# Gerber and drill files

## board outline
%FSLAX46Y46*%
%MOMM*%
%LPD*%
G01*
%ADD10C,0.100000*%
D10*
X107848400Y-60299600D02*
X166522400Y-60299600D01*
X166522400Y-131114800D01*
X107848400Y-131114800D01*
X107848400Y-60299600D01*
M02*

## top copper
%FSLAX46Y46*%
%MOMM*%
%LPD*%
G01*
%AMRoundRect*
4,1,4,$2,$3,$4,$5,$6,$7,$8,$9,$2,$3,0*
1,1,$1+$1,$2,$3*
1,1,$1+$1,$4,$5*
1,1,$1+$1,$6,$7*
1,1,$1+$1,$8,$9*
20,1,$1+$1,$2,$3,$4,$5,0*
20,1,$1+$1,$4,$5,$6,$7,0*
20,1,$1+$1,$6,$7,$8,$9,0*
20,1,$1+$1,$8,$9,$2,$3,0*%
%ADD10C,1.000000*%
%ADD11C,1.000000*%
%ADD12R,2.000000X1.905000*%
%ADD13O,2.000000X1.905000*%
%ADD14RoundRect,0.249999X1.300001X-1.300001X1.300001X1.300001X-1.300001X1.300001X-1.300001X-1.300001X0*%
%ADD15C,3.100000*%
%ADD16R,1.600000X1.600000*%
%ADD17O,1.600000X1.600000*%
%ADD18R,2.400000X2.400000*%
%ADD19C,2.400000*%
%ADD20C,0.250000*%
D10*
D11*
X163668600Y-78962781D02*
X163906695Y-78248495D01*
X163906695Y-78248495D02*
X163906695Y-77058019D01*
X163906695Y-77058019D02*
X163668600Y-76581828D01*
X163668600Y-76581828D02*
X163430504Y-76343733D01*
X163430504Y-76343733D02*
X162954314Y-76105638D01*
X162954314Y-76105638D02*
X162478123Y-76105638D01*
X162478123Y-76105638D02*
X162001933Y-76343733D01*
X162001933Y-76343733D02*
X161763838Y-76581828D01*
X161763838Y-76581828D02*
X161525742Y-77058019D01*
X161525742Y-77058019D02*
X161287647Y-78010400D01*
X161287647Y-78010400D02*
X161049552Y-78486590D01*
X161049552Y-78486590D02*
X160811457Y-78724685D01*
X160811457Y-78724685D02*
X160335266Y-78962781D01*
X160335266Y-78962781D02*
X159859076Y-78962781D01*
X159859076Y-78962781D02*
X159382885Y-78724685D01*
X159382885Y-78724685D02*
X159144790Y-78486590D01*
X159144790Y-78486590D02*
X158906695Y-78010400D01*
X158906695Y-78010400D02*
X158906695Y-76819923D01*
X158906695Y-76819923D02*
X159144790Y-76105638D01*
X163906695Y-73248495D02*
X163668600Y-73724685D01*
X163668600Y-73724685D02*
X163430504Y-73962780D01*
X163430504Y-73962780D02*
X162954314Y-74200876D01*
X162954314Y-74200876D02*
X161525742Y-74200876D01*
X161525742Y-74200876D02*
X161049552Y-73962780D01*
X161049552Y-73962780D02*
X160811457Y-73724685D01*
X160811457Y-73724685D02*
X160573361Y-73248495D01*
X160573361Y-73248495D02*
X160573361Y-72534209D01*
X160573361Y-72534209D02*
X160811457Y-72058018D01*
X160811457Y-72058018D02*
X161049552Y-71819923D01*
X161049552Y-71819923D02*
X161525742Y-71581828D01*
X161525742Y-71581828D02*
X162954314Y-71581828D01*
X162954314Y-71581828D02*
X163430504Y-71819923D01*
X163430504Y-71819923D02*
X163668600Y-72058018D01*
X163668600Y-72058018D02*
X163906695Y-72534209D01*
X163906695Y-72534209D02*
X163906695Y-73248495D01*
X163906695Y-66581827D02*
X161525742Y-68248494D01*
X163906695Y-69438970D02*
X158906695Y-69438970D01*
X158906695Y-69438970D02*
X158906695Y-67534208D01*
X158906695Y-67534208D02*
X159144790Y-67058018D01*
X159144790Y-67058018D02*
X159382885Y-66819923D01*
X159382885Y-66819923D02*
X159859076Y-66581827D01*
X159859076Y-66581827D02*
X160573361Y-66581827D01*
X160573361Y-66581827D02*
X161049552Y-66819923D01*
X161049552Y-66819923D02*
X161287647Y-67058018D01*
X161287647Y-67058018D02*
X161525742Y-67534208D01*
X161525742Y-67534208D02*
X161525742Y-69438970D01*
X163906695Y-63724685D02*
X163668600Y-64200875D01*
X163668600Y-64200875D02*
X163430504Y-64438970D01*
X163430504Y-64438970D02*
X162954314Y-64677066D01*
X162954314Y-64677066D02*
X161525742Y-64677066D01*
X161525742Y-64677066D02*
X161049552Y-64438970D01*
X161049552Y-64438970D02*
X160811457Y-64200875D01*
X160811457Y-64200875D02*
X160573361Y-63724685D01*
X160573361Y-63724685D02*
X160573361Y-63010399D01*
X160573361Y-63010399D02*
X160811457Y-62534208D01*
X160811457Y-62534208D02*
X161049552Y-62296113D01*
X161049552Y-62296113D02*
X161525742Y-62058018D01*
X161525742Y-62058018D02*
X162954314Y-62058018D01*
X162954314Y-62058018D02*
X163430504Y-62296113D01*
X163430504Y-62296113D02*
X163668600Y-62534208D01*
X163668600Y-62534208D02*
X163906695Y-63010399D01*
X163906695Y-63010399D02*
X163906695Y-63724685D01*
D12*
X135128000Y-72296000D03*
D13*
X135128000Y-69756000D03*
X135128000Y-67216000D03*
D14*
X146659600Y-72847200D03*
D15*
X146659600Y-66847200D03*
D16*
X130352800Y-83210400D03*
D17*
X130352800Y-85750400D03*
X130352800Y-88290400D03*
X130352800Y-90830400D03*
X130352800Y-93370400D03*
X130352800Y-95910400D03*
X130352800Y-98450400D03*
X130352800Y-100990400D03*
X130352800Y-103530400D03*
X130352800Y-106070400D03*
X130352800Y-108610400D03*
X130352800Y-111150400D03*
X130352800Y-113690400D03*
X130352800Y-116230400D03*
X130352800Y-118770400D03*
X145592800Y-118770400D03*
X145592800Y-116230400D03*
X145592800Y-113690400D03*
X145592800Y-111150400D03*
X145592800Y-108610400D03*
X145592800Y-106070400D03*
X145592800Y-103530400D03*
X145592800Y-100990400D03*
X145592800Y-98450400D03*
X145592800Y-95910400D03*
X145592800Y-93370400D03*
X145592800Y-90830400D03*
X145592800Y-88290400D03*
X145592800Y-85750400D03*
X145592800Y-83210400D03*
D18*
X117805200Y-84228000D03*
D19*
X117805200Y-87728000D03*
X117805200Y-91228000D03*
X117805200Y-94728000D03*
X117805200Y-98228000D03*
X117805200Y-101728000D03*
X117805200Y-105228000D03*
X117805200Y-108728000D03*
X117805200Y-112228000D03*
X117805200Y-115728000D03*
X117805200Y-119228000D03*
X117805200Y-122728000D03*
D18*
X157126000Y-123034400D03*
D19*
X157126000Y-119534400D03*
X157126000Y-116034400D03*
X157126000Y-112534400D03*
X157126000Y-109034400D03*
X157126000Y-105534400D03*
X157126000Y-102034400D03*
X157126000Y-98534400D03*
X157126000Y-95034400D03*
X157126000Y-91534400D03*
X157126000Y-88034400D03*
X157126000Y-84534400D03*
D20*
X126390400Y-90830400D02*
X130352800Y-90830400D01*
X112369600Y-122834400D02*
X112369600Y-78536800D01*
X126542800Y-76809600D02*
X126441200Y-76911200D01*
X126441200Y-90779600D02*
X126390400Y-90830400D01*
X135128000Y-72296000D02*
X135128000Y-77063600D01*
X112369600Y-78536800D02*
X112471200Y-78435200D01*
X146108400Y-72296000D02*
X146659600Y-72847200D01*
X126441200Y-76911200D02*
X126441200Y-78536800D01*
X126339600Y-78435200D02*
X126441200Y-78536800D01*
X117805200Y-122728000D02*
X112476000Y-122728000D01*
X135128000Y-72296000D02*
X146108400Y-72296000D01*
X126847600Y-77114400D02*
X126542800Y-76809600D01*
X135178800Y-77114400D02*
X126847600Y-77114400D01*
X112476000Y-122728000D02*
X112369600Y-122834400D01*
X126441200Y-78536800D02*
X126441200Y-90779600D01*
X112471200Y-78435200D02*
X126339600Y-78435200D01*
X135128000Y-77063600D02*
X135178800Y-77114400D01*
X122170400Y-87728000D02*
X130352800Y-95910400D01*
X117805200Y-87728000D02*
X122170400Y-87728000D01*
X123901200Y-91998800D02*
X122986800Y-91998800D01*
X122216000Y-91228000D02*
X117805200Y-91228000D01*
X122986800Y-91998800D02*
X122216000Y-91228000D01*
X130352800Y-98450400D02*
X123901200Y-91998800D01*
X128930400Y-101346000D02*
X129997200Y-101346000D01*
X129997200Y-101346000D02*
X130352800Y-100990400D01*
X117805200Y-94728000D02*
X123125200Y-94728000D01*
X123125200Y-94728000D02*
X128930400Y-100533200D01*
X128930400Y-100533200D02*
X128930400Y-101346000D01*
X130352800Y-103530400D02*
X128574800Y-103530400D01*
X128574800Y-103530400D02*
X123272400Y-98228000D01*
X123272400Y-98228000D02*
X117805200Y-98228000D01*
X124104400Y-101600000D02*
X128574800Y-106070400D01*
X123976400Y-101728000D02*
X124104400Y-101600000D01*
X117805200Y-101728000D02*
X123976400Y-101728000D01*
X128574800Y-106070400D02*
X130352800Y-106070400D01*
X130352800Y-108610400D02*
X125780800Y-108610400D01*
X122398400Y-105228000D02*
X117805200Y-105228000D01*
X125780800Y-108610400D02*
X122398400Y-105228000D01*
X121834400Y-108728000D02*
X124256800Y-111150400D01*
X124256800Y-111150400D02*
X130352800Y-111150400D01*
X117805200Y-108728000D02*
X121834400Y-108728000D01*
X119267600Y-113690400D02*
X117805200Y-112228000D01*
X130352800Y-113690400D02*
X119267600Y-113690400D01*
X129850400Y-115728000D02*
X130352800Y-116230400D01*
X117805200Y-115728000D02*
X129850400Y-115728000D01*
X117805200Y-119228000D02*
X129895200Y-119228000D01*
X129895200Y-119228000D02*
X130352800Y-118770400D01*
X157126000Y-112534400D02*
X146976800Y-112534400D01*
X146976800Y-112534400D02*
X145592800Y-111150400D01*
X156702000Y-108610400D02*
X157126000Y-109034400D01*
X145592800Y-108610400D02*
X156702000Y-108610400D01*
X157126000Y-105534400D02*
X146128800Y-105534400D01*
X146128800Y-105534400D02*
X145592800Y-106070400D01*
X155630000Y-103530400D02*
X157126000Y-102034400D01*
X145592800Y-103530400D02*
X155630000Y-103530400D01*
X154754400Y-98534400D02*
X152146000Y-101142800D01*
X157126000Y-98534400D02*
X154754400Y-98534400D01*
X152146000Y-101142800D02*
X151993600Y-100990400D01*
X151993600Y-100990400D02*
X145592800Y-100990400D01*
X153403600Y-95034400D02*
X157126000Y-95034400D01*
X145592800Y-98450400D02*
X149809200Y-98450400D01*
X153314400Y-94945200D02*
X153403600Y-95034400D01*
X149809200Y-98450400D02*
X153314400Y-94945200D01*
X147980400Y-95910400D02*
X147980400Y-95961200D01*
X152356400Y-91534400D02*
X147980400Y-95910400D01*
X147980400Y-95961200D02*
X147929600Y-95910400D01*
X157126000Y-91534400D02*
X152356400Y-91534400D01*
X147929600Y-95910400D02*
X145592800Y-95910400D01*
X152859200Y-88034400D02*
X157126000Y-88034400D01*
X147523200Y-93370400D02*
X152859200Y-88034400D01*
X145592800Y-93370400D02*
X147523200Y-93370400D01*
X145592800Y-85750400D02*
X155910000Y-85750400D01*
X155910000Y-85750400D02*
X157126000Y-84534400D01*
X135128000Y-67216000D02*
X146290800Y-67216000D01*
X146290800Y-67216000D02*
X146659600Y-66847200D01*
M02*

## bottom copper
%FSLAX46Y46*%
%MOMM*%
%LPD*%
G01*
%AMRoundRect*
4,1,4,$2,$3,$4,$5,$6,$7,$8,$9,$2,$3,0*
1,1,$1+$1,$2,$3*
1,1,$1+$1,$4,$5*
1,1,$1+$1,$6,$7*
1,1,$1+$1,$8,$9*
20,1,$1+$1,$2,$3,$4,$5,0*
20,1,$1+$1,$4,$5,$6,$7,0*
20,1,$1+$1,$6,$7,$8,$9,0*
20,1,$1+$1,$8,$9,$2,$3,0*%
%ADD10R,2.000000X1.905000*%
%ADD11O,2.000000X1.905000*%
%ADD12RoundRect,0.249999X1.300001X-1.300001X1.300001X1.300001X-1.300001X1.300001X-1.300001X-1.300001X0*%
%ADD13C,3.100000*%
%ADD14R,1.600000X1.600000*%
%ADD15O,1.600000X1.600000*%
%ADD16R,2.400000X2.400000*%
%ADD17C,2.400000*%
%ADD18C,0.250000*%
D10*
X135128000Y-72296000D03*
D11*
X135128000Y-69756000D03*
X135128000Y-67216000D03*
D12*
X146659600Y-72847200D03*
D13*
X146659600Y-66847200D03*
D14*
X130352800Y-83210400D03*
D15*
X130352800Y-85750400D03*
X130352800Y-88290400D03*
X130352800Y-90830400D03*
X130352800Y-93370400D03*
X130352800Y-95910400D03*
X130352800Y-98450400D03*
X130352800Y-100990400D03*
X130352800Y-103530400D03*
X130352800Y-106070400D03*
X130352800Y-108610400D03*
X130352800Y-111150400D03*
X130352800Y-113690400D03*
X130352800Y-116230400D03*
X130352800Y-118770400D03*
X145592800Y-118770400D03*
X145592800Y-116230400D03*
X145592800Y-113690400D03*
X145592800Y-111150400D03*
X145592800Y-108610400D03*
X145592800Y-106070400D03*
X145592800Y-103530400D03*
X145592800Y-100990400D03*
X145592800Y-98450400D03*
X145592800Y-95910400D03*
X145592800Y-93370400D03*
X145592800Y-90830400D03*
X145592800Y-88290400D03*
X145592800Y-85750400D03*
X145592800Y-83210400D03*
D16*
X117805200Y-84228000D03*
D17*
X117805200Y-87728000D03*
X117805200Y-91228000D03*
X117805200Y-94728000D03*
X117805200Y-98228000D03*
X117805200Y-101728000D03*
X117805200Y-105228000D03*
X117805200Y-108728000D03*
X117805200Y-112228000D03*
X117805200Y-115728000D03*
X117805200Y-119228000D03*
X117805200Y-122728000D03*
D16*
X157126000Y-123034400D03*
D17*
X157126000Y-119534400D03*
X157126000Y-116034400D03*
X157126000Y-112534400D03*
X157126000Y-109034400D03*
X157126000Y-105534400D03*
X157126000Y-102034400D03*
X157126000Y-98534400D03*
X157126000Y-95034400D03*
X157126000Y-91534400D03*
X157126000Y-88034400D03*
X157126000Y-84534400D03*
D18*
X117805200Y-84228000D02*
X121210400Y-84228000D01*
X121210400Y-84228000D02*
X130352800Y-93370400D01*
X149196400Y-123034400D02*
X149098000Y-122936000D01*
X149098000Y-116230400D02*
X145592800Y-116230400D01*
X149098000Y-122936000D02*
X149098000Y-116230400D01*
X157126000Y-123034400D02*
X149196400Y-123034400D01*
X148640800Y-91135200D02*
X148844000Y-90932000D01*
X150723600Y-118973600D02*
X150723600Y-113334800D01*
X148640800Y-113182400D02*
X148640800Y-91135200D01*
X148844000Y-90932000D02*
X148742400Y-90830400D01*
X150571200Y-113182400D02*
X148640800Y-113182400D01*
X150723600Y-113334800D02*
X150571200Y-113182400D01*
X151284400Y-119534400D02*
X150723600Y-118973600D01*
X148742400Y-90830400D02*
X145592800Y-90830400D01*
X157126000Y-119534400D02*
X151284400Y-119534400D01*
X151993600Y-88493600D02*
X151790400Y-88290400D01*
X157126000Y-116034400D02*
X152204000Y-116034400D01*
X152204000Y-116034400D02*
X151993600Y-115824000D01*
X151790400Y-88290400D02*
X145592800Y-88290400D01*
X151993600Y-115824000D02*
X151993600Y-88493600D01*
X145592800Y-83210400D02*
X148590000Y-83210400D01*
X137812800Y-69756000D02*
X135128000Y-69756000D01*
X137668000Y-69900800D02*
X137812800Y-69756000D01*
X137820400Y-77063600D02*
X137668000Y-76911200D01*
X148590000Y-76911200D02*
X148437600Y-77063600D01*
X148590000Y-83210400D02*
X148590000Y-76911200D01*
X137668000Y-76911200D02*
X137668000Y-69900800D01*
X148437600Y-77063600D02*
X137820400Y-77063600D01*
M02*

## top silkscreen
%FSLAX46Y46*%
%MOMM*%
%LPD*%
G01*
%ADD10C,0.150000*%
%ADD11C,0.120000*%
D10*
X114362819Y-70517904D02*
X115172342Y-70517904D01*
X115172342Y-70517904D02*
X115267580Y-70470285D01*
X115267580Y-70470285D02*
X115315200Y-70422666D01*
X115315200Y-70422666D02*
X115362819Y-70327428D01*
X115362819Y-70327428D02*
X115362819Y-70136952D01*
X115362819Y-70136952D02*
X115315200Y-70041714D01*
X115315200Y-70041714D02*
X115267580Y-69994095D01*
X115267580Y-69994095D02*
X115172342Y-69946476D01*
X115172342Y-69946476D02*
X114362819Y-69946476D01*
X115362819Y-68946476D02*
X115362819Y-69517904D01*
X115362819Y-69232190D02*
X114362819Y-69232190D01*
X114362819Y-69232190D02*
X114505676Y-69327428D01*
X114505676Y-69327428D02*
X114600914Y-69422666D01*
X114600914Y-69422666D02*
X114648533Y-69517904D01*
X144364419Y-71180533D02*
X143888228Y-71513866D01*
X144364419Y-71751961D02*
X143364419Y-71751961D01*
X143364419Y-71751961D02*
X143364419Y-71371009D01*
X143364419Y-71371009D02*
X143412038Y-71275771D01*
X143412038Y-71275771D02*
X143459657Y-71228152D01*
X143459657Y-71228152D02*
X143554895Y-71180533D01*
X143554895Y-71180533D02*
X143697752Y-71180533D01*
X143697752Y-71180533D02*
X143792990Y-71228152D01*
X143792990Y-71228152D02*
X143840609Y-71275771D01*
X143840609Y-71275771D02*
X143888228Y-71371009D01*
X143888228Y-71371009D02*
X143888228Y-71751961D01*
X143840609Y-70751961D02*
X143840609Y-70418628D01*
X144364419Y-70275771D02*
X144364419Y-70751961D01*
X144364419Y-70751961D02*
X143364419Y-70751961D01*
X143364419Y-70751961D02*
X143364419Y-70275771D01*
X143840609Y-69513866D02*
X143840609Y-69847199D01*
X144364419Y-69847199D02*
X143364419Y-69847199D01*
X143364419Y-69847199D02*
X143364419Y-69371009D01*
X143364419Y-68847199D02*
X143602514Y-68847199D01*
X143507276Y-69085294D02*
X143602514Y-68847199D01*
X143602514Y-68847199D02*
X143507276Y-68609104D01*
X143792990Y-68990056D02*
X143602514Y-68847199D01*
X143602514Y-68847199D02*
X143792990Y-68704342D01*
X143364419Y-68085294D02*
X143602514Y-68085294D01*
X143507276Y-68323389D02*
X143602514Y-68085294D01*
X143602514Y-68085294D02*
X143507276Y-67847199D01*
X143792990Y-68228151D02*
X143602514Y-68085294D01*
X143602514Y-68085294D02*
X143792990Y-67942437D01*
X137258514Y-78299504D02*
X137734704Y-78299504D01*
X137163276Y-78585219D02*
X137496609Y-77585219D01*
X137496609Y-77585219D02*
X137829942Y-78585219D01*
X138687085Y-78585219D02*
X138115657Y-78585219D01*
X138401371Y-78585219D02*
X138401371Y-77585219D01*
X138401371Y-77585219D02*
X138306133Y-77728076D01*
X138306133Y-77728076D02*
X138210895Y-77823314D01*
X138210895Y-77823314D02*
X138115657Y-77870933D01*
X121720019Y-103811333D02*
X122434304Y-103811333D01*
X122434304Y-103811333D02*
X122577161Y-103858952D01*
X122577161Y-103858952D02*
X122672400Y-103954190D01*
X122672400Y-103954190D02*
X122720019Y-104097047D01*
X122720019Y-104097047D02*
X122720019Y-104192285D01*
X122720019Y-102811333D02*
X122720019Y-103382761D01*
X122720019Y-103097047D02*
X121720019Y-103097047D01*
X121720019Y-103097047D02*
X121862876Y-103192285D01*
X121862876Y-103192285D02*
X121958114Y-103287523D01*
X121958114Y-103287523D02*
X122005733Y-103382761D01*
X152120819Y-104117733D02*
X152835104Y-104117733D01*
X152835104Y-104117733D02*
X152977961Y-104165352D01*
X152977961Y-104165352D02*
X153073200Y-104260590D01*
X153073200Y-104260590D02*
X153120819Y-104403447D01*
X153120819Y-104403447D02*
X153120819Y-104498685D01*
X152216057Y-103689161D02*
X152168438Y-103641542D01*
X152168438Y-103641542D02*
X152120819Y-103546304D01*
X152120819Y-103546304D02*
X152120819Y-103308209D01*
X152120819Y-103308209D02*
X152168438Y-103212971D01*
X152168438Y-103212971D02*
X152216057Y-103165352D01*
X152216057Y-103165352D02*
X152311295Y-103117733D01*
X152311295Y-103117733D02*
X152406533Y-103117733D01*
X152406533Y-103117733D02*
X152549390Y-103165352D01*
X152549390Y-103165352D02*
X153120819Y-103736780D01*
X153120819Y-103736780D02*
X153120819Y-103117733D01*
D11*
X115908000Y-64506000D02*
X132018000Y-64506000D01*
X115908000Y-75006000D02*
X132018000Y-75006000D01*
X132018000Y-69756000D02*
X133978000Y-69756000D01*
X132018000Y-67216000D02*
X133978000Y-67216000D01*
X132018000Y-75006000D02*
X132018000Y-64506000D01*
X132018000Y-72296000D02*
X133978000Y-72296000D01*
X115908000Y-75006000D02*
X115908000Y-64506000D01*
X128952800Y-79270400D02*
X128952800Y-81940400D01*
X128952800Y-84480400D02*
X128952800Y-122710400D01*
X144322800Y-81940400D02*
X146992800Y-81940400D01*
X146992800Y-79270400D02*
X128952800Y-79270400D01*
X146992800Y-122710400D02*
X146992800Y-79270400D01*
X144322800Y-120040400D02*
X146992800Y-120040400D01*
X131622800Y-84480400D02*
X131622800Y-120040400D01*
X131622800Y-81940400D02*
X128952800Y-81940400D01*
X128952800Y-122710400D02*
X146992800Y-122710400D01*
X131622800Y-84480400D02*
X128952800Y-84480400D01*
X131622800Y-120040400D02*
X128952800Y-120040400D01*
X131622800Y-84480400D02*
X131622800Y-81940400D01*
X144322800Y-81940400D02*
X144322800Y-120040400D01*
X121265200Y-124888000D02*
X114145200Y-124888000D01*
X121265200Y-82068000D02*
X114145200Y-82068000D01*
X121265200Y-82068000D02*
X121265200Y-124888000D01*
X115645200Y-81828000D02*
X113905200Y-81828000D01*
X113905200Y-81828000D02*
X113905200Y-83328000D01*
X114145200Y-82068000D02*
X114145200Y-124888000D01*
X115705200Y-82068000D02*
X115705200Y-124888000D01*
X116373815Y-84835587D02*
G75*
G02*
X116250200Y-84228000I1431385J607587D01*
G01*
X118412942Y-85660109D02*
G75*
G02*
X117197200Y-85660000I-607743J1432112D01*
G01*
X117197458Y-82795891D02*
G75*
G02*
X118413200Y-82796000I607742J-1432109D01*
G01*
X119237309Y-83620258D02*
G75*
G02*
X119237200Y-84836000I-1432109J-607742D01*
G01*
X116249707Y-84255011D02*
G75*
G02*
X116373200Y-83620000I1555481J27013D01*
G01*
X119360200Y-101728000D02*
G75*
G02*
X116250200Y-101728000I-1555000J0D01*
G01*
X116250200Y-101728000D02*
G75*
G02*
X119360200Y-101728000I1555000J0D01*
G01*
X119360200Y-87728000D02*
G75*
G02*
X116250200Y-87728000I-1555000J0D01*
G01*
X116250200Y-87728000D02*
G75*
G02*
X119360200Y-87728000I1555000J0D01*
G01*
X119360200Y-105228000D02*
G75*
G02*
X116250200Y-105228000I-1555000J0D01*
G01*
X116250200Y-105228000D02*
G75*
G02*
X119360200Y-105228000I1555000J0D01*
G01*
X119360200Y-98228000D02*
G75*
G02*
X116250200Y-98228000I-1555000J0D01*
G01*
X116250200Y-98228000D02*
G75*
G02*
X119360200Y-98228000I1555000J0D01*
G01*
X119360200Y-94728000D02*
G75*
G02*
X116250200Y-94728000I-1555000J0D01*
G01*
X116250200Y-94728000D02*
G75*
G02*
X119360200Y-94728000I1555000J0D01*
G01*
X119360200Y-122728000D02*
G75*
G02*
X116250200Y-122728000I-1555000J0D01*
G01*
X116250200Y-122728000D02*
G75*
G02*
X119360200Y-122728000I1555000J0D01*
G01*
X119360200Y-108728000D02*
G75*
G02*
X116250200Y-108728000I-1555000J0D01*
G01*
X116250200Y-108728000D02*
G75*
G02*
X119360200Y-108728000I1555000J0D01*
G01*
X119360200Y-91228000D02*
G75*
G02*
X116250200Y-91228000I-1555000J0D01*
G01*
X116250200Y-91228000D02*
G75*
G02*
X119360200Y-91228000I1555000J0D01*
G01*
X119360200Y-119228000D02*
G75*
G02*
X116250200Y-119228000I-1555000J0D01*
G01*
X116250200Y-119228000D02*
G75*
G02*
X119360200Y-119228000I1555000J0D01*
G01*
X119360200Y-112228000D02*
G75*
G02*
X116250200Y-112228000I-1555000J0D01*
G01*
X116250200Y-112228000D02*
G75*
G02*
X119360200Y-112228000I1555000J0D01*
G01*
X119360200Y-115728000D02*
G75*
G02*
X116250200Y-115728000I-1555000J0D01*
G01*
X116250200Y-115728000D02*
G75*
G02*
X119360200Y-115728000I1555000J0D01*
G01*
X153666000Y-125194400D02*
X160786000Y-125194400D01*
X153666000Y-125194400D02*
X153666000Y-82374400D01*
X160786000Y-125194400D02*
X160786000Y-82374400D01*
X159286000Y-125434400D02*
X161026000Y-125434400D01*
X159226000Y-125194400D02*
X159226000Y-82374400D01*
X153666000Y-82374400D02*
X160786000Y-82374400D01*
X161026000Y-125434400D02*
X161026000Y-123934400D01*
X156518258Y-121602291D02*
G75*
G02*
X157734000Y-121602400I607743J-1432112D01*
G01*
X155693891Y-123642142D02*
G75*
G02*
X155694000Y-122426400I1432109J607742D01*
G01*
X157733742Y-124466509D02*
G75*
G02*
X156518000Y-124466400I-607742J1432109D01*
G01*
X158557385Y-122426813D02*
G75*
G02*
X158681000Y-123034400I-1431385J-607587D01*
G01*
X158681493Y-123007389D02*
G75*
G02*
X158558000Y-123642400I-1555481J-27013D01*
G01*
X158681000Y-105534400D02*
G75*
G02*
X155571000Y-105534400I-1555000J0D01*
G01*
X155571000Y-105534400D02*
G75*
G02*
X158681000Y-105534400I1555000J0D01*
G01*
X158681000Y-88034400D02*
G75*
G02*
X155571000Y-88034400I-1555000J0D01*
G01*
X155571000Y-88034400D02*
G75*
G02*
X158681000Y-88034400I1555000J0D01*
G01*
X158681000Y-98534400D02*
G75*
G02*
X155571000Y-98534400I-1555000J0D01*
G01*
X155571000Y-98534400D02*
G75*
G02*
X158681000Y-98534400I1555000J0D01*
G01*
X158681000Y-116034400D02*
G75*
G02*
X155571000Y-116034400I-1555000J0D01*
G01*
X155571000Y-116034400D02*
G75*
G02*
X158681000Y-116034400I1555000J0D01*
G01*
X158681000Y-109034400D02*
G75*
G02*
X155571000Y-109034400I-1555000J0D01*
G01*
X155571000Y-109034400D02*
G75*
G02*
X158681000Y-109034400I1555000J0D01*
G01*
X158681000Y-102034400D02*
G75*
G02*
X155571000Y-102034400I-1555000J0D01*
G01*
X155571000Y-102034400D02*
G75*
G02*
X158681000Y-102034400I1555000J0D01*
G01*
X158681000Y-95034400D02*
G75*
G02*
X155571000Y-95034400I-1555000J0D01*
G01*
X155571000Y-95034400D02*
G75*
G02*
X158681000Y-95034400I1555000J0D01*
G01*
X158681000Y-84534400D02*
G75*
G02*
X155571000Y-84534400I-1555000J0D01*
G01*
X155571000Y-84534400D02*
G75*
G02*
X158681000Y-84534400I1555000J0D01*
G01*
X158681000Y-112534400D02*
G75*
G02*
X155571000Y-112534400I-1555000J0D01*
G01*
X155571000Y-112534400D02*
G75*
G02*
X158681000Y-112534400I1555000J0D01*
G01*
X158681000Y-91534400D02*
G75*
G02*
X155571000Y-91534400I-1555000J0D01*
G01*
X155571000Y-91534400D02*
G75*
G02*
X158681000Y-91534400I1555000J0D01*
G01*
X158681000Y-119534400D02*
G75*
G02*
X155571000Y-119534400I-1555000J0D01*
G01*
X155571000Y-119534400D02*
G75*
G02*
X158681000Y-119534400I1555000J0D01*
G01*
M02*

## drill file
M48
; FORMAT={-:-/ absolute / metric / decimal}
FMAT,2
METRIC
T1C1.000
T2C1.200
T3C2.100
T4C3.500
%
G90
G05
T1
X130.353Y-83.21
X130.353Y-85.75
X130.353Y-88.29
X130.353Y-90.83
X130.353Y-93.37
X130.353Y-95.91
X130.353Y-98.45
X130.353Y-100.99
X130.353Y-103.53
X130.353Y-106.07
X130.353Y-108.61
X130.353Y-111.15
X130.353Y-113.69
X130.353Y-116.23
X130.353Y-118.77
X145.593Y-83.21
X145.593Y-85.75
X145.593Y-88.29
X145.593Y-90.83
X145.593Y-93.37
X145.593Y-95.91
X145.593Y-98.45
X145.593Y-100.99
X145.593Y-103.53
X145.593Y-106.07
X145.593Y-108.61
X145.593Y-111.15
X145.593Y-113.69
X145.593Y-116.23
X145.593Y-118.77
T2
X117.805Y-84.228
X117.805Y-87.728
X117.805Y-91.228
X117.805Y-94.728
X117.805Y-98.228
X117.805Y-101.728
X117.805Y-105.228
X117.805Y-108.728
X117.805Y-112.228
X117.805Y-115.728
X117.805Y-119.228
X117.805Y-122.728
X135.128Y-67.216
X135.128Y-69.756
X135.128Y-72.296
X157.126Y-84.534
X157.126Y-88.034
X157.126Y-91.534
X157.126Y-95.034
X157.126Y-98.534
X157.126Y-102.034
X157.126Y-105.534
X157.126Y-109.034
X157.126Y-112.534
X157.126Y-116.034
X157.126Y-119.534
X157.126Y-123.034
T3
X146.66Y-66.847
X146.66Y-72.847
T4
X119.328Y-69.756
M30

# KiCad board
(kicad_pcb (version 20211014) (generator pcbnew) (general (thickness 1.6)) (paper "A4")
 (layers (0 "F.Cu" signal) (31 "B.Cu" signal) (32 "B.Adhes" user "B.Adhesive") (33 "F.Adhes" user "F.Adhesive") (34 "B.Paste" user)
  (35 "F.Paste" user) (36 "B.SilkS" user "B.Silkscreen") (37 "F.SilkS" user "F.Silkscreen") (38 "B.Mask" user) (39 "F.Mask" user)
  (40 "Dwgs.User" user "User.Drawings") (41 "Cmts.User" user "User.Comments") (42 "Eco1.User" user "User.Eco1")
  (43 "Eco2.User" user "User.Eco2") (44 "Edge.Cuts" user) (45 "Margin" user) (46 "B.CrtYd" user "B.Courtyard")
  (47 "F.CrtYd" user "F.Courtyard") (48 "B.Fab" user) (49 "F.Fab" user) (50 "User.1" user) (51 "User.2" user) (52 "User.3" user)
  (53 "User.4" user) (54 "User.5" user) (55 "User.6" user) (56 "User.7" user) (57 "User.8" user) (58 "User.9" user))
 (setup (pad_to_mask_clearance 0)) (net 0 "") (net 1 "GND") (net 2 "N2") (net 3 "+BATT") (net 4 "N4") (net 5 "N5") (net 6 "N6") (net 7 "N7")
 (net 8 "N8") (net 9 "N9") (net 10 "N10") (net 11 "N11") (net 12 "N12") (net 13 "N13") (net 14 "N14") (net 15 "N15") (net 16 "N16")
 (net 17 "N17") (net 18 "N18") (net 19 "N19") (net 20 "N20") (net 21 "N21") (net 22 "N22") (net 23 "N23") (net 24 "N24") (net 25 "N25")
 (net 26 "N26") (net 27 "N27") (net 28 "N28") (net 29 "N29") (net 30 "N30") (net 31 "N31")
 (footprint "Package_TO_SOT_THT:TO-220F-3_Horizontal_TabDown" (layer "F.Cu") (at 135.128 72.296 90)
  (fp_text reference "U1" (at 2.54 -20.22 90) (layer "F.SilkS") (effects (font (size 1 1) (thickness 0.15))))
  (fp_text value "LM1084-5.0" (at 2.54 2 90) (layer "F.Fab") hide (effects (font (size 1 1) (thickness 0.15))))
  (fp_line (start 7.79 -19.22) (end 7.79 -3.11) (layer "F.SilkS") (width 0.12))
  (fp_line (start -2.71 -19.22) (end -2.71 -3.11) (layer "F.SilkS") (width 0.12))
  (fp_line (start 2.54 -3.11) (end 2.54 -1.15) (layer "F.SilkS") (width 0.12))
  (fp_line (start 5.08 -3.11) (end 5.08 -1.15) (layer "F.SilkS") (width 0.12))
  (fp_line (start -2.71 -3.11) (end 7.79 -3.11) (layer "F.SilkS") (width 0.12))
  (fp_line (start 0 -3.11) (end 0 -1.15) (layer "F.SilkS") (width 0.12))
  (fp_line (start -2.71 -19.22) (end 7.79 -19.22) (layer "F.SilkS") (width 0.12))
  (pad "" np_thru_hole oval (at 2.54 -15.8 90) (size 3.5 3.5) (drill 3.5) (layers *.Cu *.Mask))
  (pad "1" thru_hole rect (at 0 0 90) (size 1.905 2) (drill 1.2) (layers *.Cu *.Mask) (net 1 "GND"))
  (pad "2" thru_hole oval (at 2.54 0 90) (size 1.905 2) (drill 1.2) (layers *.Cu *.Mask) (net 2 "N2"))
  (pad "3" thru_hole oval (at 5.08 0 90) (size 1.905 2) (drill 1.2) (layers *.Cu *.Mask) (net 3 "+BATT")))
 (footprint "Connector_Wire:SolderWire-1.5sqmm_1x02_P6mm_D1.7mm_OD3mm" (layer "F.Cu") (at 146.6596 72.8472 90)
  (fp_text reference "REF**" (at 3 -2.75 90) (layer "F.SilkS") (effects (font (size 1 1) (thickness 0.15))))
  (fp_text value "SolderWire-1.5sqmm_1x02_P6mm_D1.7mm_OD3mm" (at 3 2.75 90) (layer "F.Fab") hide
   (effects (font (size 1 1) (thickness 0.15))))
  (pad "1" thru_hole roundrect (at 0 0 90) (size 3.1 3.1) (drill 2.1) (layers *.Cu *.Mask) (roundrect_rratio 0.08064483871) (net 1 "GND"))
  (pad "2" thru_hole circle (at 6 0 90) (size 3.1 3.1) (drill 2.1) (layers *.Cu *.Mask) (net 3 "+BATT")))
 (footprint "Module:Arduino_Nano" (layer "F.Cu") (at 130.3528 83.2104)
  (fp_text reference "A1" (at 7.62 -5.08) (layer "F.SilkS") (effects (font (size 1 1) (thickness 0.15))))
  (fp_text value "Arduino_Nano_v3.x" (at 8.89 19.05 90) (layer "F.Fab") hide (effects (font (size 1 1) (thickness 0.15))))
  (fp_line (start -1.4 -3.94) (end -1.4 -1.27) (layer "F.SilkS") (width 0.12))
  (fp_line (start -1.4 1.27) (end -1.4 39.5) (layer "F.SilkS") (width 0.12))
  (fp_line (start 13.97 -1.27) (end 16.64 -1.27) (layer "F.SilkS") (width 0.12))
  (fp_line (start 16.64 -3.94) (end -1.4 -3.94) (layer "F.SilkS") (width 0.12))
  (fp_line (start 16.64 39.5) (end 16.64 -3.94) (layer "F.SilkS") (width 0.12))
  (fp_line (start 13.97 36.83) (end 16.64 36.83) (layer "F.SilkS") (width 0.12))
  (fp_line (start 1.27 1.27) (end 1.27 36.83) (layer "F.SilkS") (width 0.12))
  (fp_line (start 1.27 -1.27) (end -1.4 -1.27) (layer "F.SilkS") (width 0.12))
  (fp_line (start -1.4 39.5) (end 16.64 39.5) (layer "F.SilkS") (width 0.12))
  (fp_line (start 1.27 1.27) (end -1.4 1.27) (layer "F.SilkS") (width 0.12))
  (fp_line (start 1.27 36.83) (end -1.4 36.83) (layer "F.SilkS") (width 0.12))
  (fp_line (start 1.27 1.27) (end 1.27 -1.27) (layer "F.SilkS") (width 0.12))
  (fp_line (start 13.97 -1.27) (end 13.97 36.83) (layer "F.SilkS") (width 0.12))
  (pad "1" thru_hole rect (at 0 0) (size 1.6 1.6) (drill 1) (layers *.Cu *.Mask) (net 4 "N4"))
  (pad "2" thru_hole oval (at 0 2.54) (size 1.6 1.6) (drill 1) (layers *.Cu *.Mask) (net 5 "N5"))
  (pad "3" thru_hole oval (at 0 5.08) (size 1.6 1.6) (drill 1) (layers *.Cu *.Mask) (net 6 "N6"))
  (pad "4" thru_hole oval (at 0 7.62) (size 1.6 1.6) (drill 1) (layers *.Cu *.Mask) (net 1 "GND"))
  (pad "5" thru_hole oval (at 0 10.16) (size 1.6 1.6) (drill 1) (layers *.Cu *.Mask) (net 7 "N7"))
  (pad "6" thru_hole oval (at 0 12.7) (size 1.6 1.6) (drill 1) (layers *.Cu *.Mask) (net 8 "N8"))
  (pad "7" thru_hole oval (at 0 15.24) (size 1.6 1.6) (drill 1) (layers *.Cu *.Mask) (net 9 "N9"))
  (pad "8" thru_hole oval (at 0 17.78) (size 1.6 1.6) (drill 1) (layers *.Cu *.Mask) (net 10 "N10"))
  (pad "9" thru_hole oval (at 0 20.32) (size 1.6 1.6) (drill 1) (layers *.Cu *.Mask) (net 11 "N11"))
  (pad "10" thru_hole oval (at 0 22.86) (size 1.6 1.6) (drill 1) (layers *.Cu *.Mask) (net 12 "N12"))
  (pad "11" thru_hole oval (at 0 25.4) (size 1.6 1.6) (drill 1) (layers *.Cu *.Mask) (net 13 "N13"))
  (pad "12" thru_hole oval (at 0 27.94) (size 1.6 1.6) (drill 1) (layers *.Cu *.Mask) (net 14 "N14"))
  (pad "13" thru_hole oval (at 0 30.48) (size 1.6 1.6) (drill 1) (layers *.Cu *.Mask) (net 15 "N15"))
  (pad "14" thru_hole oval (at 0 33.02) (size 1.6 1.6) (drill 1) (layers *.Cu *.Mask) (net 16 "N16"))
  (pad "15" thru_hole oval (at 0 35.56) (size 1.6 1.6) (drill 1) (layers *.Cu *.Mask) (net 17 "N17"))
  (pad "16" thru_hole oval (at 15.24 35.56) (size 1.6 1.6) (drill 1) (layers *.Cu *.Mask) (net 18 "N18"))
  (pad "17" thru_hole oval (at 15.24 33.02) (size 1.6 1.6) (drill 1) (layers *.Cu *.Mask) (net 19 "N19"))
  (pad "18" thru_hole oval (at 15.24 30.48) (size 1.6 1.6) (drill 1) (layers *.Cu *.Mask) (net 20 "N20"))
  (pad "19" thru_hole oval (at 15.24 27.94) (size 1.6 1.6) (drill 1) (layers *.Cu *.Mask) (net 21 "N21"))
  (pad "20" thru_hole oval (at 15.24 25.4) (size 1.6 1.6) (drill 1) (layers *.Cu *.Mask) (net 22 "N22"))
  (pad "21" thru_hole oval (at 15.24 22.86) (size 1.6 1.6) (drill 1) (layers *.Cu *.Mask) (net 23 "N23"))
  (pad "22" thru_hole oval (at 15.24 20.32) (size 1.6 1.6) (drill 1) (layers *.Cu *.Mask) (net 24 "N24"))
  (pad "23" thru_hole oval (at 15.24 17.78) (size 1.6 1.6) (drill 1) (layers *.Cu *.Mask) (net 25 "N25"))
  (pad "24" thru_hole oval (at 15.24 15.24) (size 1.6 1.6) (drill 1) (layers *.Cu *.Mask) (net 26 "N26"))
  (pad "25" thru_hole oval (at 15.24 12.7) (size 1.6 1.6) (drill 1) (layers *.Cu *.Mask) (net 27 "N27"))
  (pad "26" thru_hole oval (at 15.24 10.16) (size 1.6 1.6) (drill 1) (layers *.Cu *.Mask) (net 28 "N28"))
  (pad "27" thru_hole oval (at 15.24 7.62) (size 1.6 1.6) (drill 1) (layers *.Cu *.Mask) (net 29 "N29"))
  (pad "28" thru_hole oval (at 15.24 5.08) (size 1.6 1.6) (drill 1) (layers *.Cu *.Mask) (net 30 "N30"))
  (pad "29" thru_hole oval (at 15.24 2.54) (size 1.6 1.6) (drill 1) (layers *.Cu *.Mask) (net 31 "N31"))
  (pad "30" thru_hole oval (at 15.24 0) (size 1.6 1.6) (drill 1) (layers *.Cu *.Mask) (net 2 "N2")))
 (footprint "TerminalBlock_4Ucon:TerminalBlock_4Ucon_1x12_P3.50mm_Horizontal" (layer "F.Cu") (at 117.8052 84.228 -90)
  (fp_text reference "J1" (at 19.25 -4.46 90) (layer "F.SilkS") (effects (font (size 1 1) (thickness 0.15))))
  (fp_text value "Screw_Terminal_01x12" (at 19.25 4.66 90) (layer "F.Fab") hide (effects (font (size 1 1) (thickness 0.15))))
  (fp_line (start 40.66 -3.46) (end 40.66 3.66) (layer "F.SilkS") (width 0.12))
  (fp_line (start -2.16 -3.46) (end -2.16 3.66) (layer "F.SilkS") (width 0.12))
  (fp_line (start -2.16 -3.46) (end 40.66 -3.46) (layer "F.SilkS") (width 0.12))
  (fp_line (start -2.4 2.16) (end -2.4 3.9) (layer "F.SilkS") (width 0.12))
  (fp_line (start -2.4 3.9) (end -0.9 3.9) (layer "F.SilkS") (width 0.12))
  (fp_line (start -2.16 3.66) (end 40.66 3.66) (layer "F.SilkS") (width 0.12))
  (fp_line (start -2.16 2.1) (end 40.66 2.1) (layer "F.SilkS") (width 0.12))
  (fp_arc (start 0.607587 1.431385) (mid 0.310017 1.523783) (end 0 1.555) (layer "F.SilkS") (width 0.12))
  (fp_arc (start 1.432109 -0.607742) (mid 1.555727 0.00014) (end 1.432 0.608) (layer "F.SilkS") (width 0.12))
  (fp_arc (start -1.432109 0.607742) (mid -1.555727 -0.00014) (end -1.432 -0.608) (layer "F.SilkS") (width 0.12))
  (fp_arc (start -0.607742 -1.432109) (mid 0.00014 -1.555727) (end 0.608 -1.432) (layer "F.SilkS") (width 0.12))
  (fp_arc (start 0.027011 1.555493) (mid -0.296984 1.527118) (end -0.608 1.432) (layer "F.SilkS") (width 0.12))
  (fp_circle (center 17.5 0) (end 19.055 0) (layer "F.SilkS") (width 0.12) (fill none))
  (fp_circle (center 3.5 0) (end 5.055 0) (layer "F.SilkS") (width 0.12) (fill none))
  (fp_circle (center 21 0) (end 22.555 0) (layer "F.SilkS") (width 0.12) (fill none))
  (fp_circle (center 14 0) (end 15.555 0) (layer "F.SilkS") (width 0.12) (fill none))
  (fp_circle (center 10.5 0) (end 12.055 0) (layer "F.SilkS") (width 0.12) (fill none))
  (fp_circle (center 38.5 0) (end 40.055 0) (layer "F.SilkS") (width 0.12) (fill none))
  (fp_circle (center 24.5 0) (end 26.055 0) (layer "F.SilkS") (width 0.12) (fill none))
  (fp_circle (center 7 0) (end 8.555 0) (layer "F.SilkS") (width 0.12) (fill none))
  (fp_circle (center 35 0) (end 36.555 0) (layer "F.SilkS") (width 0.12) (fill none))
  (fp_circle (center 28 0) (end 29.555 0) (layer "F.SilkS") (width 0.12) (fill none))
  (fp_circle (center 31.5 0) (end 33.055 0) (layer "F.SilkS") (width 0.12) (fill none))
  (pad "1" thru_hole rect (at 0 0 270) (size 2.4 2.4) (drill 1.2) (layers *.Cu *.Mask) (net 7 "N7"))
  (pad "2" thru_hole circle (at 3.5 0 270) (size 2.4 2.4) (drill 1.2) (layers *.Cu *.Mask) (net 8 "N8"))
  (pad "3" thru_hole circle (at 7 0 270) (size 2.4 2.4) (drill 1.2) (layers *.Cu *.Mask) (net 9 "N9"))
  (pad "4" thru_hole circle (at 10.5 0 270) (size 2.4 2.4) (drill 1.2) (layers *.Cu *.Mask) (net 10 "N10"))
  (pad "5" thru_hole circle (at 14 0 270) (size 2.4 2.4) (drill 1.2) (layers *.Cu *.Mask) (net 11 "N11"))
  (pad "6" thru_hole circle (at 17.5 0 270) (size 2.4 2.4) (drill 1.2) (layers *.Cu *.Mask) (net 12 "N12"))
  (pad "7" thru_hole circle (at 21 0 270) (size 2.4 2.4) (drill 1.2) (layers *.Cu *.Mask) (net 13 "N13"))
  (pad "8" thru_hole circle (at 24.5 0 270) (size 2.4 2.4) (drill 1.2) (layers *.Cu *.Mask) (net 14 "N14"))
  (pad "9" thru_hole circle (at 28 0 270) (size 2.4 2.4) (drill 1.2) (layers *.Cu *.Mask) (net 15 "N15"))
  (pad "10" thru_hole circle (at 31.5 0 270) (size 2.4 2.4) (drill 1.2) (layers *.Cu *.Mask) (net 16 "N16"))
  (pad "11" thru_hole circle (at 35 0 270) (size 2.4 2.4) (drill 1.2) (layers *.Cu *.Mask) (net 17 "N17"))
  (pad "12" thru_hole circle (at 38.5 0 270) (size 2.4 2.4) (drill 1.2) (layers *.Cu *.Mask) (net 1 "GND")))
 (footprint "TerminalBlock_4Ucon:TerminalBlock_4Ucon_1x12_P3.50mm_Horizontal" (layer "F.Cu") (at 157.126 123.0344 90)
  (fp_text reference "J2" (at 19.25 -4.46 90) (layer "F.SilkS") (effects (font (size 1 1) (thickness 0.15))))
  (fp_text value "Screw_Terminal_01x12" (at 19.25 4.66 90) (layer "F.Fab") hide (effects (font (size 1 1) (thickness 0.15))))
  (fp_line (start -2.16 -3.46) (end -2.16 3.66) (layer "F.SilkS") (width 0.12))
  (fp_line (start -2.16 -3.46) (end 40.66 -3.46) (layer "F.SilkS") (width 0.12))
  (fp_line (start -2.16 3.66) (end 40.66 3.66) (layer "F.SilkS") (width 0.12))
  (fp_line (start -2.4 2.16) (end -2.4 3.9) (layer "F.SilkS") (width 0.12))
  (fp_line (start -2.16 2.1) (end 40.66 2.1) (layer "F.SilkS") (width 0.12))
  (fp_line (start 40.66 -3.46) (end 40.66 3.66) (layer "F.SilkS") (width 0.12))
  (fp_line (start -2.4 3.9) (end -0.9 3.9) (layer "F.SilkS") (width 0.12))
  (fp_arc (start 1.432109 -0.607742) (mid 1.555727 0.00014) (end 1.432 0.608) (layer "F.SilkS") (width 0.12))
  (fp_arc (start -0.607742 -1.432109) (mid 0.00014 -1.555727) (end 0.608 -1.432) (layer "F.SilkS") (width 0.12))
  (fp_arc (start -1.432109 0.607742) (mid -1.555727 -0.00014) (end -1.432 -0.608) (layer "F.SilkS") (width 0.12))
  (fp_arc (start 0.607587 1.431385) (mid 0.310017 1.523783) (end 0 1.555) (layer "F.SilkS") (width 0.12))
  (fp_arc (start 0.027011 1.555493) (mid -0.296984 1.527118) (end -0.608 1.432) (layer "F.SilkS") (width 0.12))
  (fp_circle (center 17.5 0) (end 19.055 0) (layer "F.SilkS") (width 0.12) (fill none))
  (fp_circle (center 35 0) (end 36.555 0) (layer "F.SilkS") (width 0.12) (fill none))
  (fp_circle (center 24.5 0) (end 26.055 0) (layer "F.SilkS") (width 0.12) (fill none))
  (fp_circle (center 7 0) (end 8.555 0) (layer "F.SilkS") (width 0.12) (fill none))
  (fp_circle (center 14 0) (end 15.555 0) (layer "F.SilkS") (width 0.12) (fill none))
  (fp_circle (center 21 0) (end 22.555 0) (layer "F.SilkS") (width 0.12) (fill none))
  (fp_circle (center 28 0) (end 29.555 0) (layer "F.SilkS") (width 0.12) (fill none))
  (fp_circle (center 38.5 0) (end 40.055 0) (layer "F.SilkS") (width 0.12) (fill none))
  (fp_circle (center 10.5 0) (end 12.055 0) (layer "F.SilkS") (width 0.12) (fill none))
  (fp_circle (center 31.5 0) (end 33.055 0) (layer "F.SilkS") (width 0.12) (fill none))
  (fp_circle (center 3.5 0) (end 5.055 0) (layer "F.SilkS") (width 0.12) (fill none))
  (pad "1" thru_hole rect (at 0 0 90) (size 2.4 2.4) (drill 1.2) (layers *.Cu *.Mask) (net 19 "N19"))
  (pad "2" thru_hole circle (at 3.5 0 90) (size 2.4 2.4) (drill 1.2) (layers *.Cu *.Mask) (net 29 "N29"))
  (pad "3" thru_hole circle (at 7 0 90) (size 2.4 2.4) (drill 1.2) (layers *.Cu *.Mask) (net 30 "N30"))
  (pad "4" thru_hole circle (at 10.5 0 90) (size 2.4 2.4) (drill 1.2) (layers *.Cu *.Mask) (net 21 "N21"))
  (pad "5" thru_hole circle (at 14 0 90) (size 2.4 2.4) (drill 1.2) (layers *.Cu *.Mask) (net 22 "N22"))
  (pad "6" thru_hole circle (at 17.5 0 90) (size 2.4 2.4) (drill 1.2) (layers *.Cu *.Mask) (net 23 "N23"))
  (pad "7" thru_hole circle (at 21 0 90) (size 2.4 2.4) (drill 1.2) (layers *.Cu *.Mask) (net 24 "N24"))
  (pad "8" thru_hole circle (at 24.5 0 90) (size 2.4 2.4) (drill 1.2) (layers *.Cu *.Mask) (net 25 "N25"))
  (pad "9" thru_hole circle (at 28 0 90) (size 2.4 2.4) (drill 1.2) (layers *.Cu *.Mask) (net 26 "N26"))
  (pad "10" thru_hole circle (at 31.5 0 90) (size 2.4 2.4) (drill 1.2) (layers *.Cu *.Mask) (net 27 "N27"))
  (pad "11" thru_hole circle (at 35 0 90) (size 2.4 2.4) (drill 1.2) (layers *.Cu *.Mask) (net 28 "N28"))
  (pad "12" thru_hole circle (at 38.5 0 90) (size 2.4 2.4) (drill 1.2) (layers *.Cu *.Mask) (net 31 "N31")))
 (gr_rect (start 166.5224 131.1148) (end 107.8484 60.2996) (layer "Edge.Cuts") (width 0.1) (fill none))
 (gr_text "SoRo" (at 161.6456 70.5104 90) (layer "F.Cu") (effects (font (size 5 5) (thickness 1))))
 (segment (start 126.3904 90.8304) (end 130.3528 90.8304) (width 0.25) (layer "F.Cu") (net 1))
 (segment (start 112.3696 122.8344) (end 112.3696 78.5368) (width 0.25) (layer "F.Cu") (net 1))
 (segment (start 126.5428 76.8096) (end 126.4412 76.9112) (width 0.25) (layer "F.Cu") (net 1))
 (segment (start 126.4412 90.7796) (end 126.3904 90.8304) (width 0.25) (layer "F.Cu") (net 1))
 (segment (start 135.128 72.296) (end 135.128 77.0636) (width 0.25) (layer "F.Cu") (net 1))
 (segment (start 112.3696 78.5368) (end 112.4712 78.4352) (width 0.25) (layer "F.Cu") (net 1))
 (segment (start 146.1084 72.296) (end 146.6596 72.8472) (width 0.25) (layer "F.Cu") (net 1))
 (segment (start 126.4412 76.9112) (end 126.4412 78.5368) (width 0.25) (layer "F.Cu") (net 1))
 (segment (start 126.3396 78.4352) (end 126.4412 78.5368) (width 0.25) (layer "F.Cu") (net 1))
 (segment (start 117.8052 122.728) (end 112.476 122.728) (width 0.25) (layer "F.Cu") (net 1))
 (segment (start 135.128 72.296) (end 146.1084 72.296) (width 0.25) (layer "F.Cu") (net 1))
 (segment (start 126.8476 77.1144) (end 126.5428 76.8096) (width 0.25) (layer "F.Cu") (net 1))
 (segment (start 135.1788 77.1144) (end 126.8476 77.1144) (width 0.25) (layer "F.Cu") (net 1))
 (segment (start 112.476 122.728) (end 112.3696 122.8344) (width 0.25) (layer "F.Cu") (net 1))
 (segment (start 126.4412 78.5368) (end 126.4412 90.7796) (width 0.25) (layer "F.Cu") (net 1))
 (segment (start 112.4712 78.4352) (end 126.3396 78.4352) (width 0.25) (layer "F.Cu") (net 1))
 (segment (start 135.128 77.0636) (end 135.1788 77.1144) (width 0.25) (layer "F.Cu") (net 1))
 (segment (start 117.8052 84.228) (end 121.2104 84.228) (width 0.25) (layer "B.Cu") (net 7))
 (segment (start 121.2104 84.228) (end 130.3528 93.3704) (width 0.25) (layer "B.Cu") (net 7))
 (segment (start 122.1704 87.728) (end 130.3528 95.9104) (width 0.25) (layer "F.Cu") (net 8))
 (segment (start 117.8052 87.728) (end 122.1704 87.728) (width 0.25) (layer "F.Cu") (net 8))
 (segment (start 123.9012 91.9988) (end 122.9868 91.9988) (width 0.25) (layer "F.Cu") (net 9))
 (segment (start 122.216 91.228) (end 117.8052 91.228) (width 0.25) (layer "F.Cu") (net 9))
 (segment (start 122.9868 91.9988) (end 122.216 91.228) (width 0.25) (layer "F.Cu") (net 9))
 (segment (start 130.3528 98.4504) (end 123.9012 91.9988) (width 0.25) (layer "F.Cu") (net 9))
 (segment (start 128.9304 101.346) (end 129.9972 101.346) (width 0.25) (layer "F.Cu") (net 10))
 (segment (start 129.9972 101.346) (end 130.3528 100.9904) (width 0.25) (layer "F.Cu") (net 10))
 (segment (start 117.8052 94.728) (end 123.1252 94.728) (width 0.25) (layer "F.Cu") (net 10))
 (segment (start 123.1252 94.728) (end 128.9304 100.5332) (width 0.25) (layer "F.Cu") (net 10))
 (segment (start 128.9304 100.5332) (end 128.9304 101.346) (width 0.25) (layer "F.Cu") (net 10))
 (segment (start 130.3528 103.5304) (end 128.5748 103.5304) (width 0.25) (layer "F.Cu") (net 11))
 (segment (start 128.5748 103.5304) (end 123.2724 98.228) (width 0.25) (layer "F.Cu") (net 11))
 (segment (start 123.2724 98.228) (end 117.8052 98.228) (width 0.25) (layer "F.Cu") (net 11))
 (segment (start 124.1044 101.6) (end 128.5748 106.0704) (width 0.25) (layer "F.Cu") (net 12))
 (segment (start 123.9764 101.728) (end 124.1044 101.6) (width 0.25) (layer "F.Cu") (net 12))
 (segment (start 117.8052 101.728) (end 123.9764 101.728) (width 0.25) (layer "F.Cu") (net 12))
 (segment (start 128.5748 106.0704) (end 130.3528 106.0704) (width 0.25) (layer "F.Cu") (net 12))
 (segment (start 130.3528 108.6104) (end 125.7808 108.6104) (width 0.25) (layer "F.Cu") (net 13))
 (segment (start 122.3984 105.228) (end 117.8052 105.228) (width 0.25) (layer "F.Cu") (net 13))
 (segment (start 125.7808 108.6104) (end 122.3984 105.228) (width 0.25) (layer "F.Cu") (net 13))
 (segment (start 121.8344 108.728) (end 124.2568 111.1504) (width 0.25) (layer "F.Cu") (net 14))
 (segment (start 124.2568 111.1504) (end 130.3528 111.1504) (width 0.25) (layer "F.Cu") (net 14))
 (segment (start 117.8052 108.728) (end 121.8344 108.728) (width 0.25) (layer "F.Cu") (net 14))
 (segment (start 119.2676 113.6904) (end 117.8052 112.228) (width 0.25) (layer "F.Cu") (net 15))
 (segment (start 130.3528 113.6904) (end 119.2676 113.6904) (width 0.25) (layer "F.Cu") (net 15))
 (segment (start 129.8504 115.728) (end 130.3528 116.2304) (width 0.25) (layer "F.Cu") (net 16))
 (segment (start 117.8052 115.728) (end 129.8504 115.728) (width 0.25) (layer "F.Cu") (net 16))
 (segment (start 117.8052 119.228) (end 129.8952 119.228) (width 0.25) (layer "F.Cu") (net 17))
 (segment (start 129.8952 119.228) (end 130.3528 118.7704) (width 0.25) (layer "F.Cu") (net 17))
 (segment (start 149.1964 123.0344) (end 149.098 122.936) (width 0.25) (layer "B.Cu") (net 19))
 (segment (start 149.098 116.2304) (end 145.5928 116.2304) (width 0.25) (layer "B.Cu") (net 19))
 (segment (start 149.098 122.936) (end 149.098 116.2304) (width 0.25) (layer "B.Cu") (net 19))
 (segment (start 157.126 123.0344) (end 149.1964 123.0344) (width 0.25) (layer "B.Cu") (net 19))
 (segment (start 157.126 112.5344) (end 146.9768 112.5344) (width 0.25) (layer "F.Cu") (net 21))
 (segment (start 146.9768 112.5344) (end 145.5928 111.1504) (width 0.25) (layer "F.Cu") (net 21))
 (segment (start 156.702 108.6104) (end 157.126 109.0344) (width 0.25) (layer "F.Cu") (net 22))
 (segment (start 145.5928 108.6104) (end 156.702 108.6104) (width 0.25) (layer "F.Cu") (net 22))
 (segment (start 157.126 105.5344) (end 146.1288 105.5344) (width 0.25) (layer "F.Cu") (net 23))
 (segment (start 146.1288 105.5344) (end 145.5928 106.0704) (width 0.25) (layer "F.Cu") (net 23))
 (segment (start 155.63 103.5304) (end 157.126 102.0344) (width 0.25) (layer "F.Cu") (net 24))
 (segment (start 145.5928 103.5304) (end 155.63 103.5304) (width 0.25) (layer "F.Cu") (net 24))
 (segment (start 154.7544 98.5344) (end 152.146 101.1428) (width 0.25) (layer "F.Cu") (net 25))
 (segment (start 157.126 98.5344) (end 154.7544 98.5344) (width 0.25) (layer "F.Cu") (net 25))
 (segment (start 152.146 101.1428) (end 151.9936 100.9904) (width 0.25) (layer "F.Cu") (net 25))
 (segment (start 151.9936 100.9904) (end 145.5928 100.9904) (width 0.25) (layer "F.Cu") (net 25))
 (segment (start 153.4036 95.0344) (end 157.126 95.0344) (width 0.25) (layer "F.Cu") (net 26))
 (segment (start 145.5928 98.4504) (end 149.8092 98.4504) (width 0.25) (layer "F.Cu") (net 26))
 (segment (start 153.3144 94.9452) (end 153.4036 95.0344) (width 0.25) (layer "F.Cu") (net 26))
 (segment (start 149.8092 98.4504) (end 153.3144 94.9452) (width 0.25) (layer "F.Cu") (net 26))
 (segment (start 147.9804 95.9104) (end 147.9804 95.9612) (width 0.25) (layer "F.Cu") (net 27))
 (segment (start 152.3564 91.5344) (end 147.9804 95.9104) (width 0.25) (layer "F.Cu") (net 27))
 (segment (start 147.9804 95.9612) (end 147.9296 95.9104) (width 0.25) (layer "F.Cu") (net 27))
 (segment (start 157.126 91.5344) (end 152.3564 91.5344) (width 0.25) (layer "F.Cu") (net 27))
 (segment (start 147.9296 95.9104) (end 145.5928 95.9104) (width 0.25) (layer "F.Cu") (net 27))
 (segment (start 152.8592 88.0344) (end 157.126 88.0344) (width 0.25) (layer "F.Cu") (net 28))
 (segment (start 147.5232 93.3704) (end 152.8592 88.0344) (width 0.25) (layer "F.Cu") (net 28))
 (segment (start 145.5928 93.3704) (end 147.5232 93.3704) (width 0.25) (layer "F.Cu") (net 28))
 (segment (start 148.6408 91.1352) (end 148.844 90.932) (width 0.25) (layer "B.Cu") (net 29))
 (segment (start 150.7236 118.9736) (end 150.7236 113.3348) (width 0.25) (layer "B.Cu") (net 29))
 (segment (start 148.6408 113.1824) (end 148.6408 91.1352) (width 0.25) (layer "B.Cu") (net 29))
 (segment (start 148.844 90.932) (end 148.7424 90.8304) (width 0.25) (layer "B.Cu") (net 29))
 (segment (start 150.5712 113.1824) (end 148.6408 113.1824) (width 0.25) (layer "B.Cu") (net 29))
 (segment (start 150.7236 113.3348) (end 150.5712 113.1824) (width 0.25) (layer "B.Cu") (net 29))
 (segment (start 151.2844 119.5344) (end 150.7236 118.9736) (width 0.25) (layer "B.Cu") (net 29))
 (segment (start 148.7424 90.8304) (end 145.5928 90.8304) (width 0.25) (layer "B.Cu") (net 29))
 (segment (start 157.126 119.5344) (end 151.2844 119.5344) (width 0.25) (layer "B.Cu") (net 29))
 (segment (start 151.9936 88.4936) (end 151.7904 88.2904) (width 0.25) (layer "B.Cu") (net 30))
 (segment (start 157.126 116.0344) (end 152.204 116.0344) (width 0.25) (layer "B.Cu") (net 30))
 (segment (start 152.204 116.0344) (end 151.9936 115.824) (width 0.25) (layer "B.Cu") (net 30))
 (segment (start 151.7904 88.2904) (end 145.5928 88.2904) (width 0.25) (layer "B.Cu") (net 30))
 (segment (start 151.9936 115.824) (end 151.9936 88.4936) (width 0.25) (layer "B.Cu") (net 30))
 (segment (start 145.5928 85.7504) (end 155.91 85.7504) (width 0.25) (layer "F.Cu") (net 31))
 (segment (start 155.91 85.7504) (end 157.126 84.5344) (width 0.25) (layer "F.Cu") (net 31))
 (segment (start 145.5928 83.2104) (end 148.59 83.2104) (width 0.25) (layer "B.Cu") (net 2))
 (segment (start 137.8128 69.756) (end 135.128 69.756) (width 0.25) (layer "B.Cu") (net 2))
 (segment (start 137.668 69.9008) (end 137.8128 69.756) (width 0.25) (layer "B.Cu") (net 2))
 (segment (start 137.8204 77.0636) (end 137.668 76.9112) (width 0.25) (layer "B.Cu") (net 2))
 (segment (start 148.59 76.9112) (end 148.4376 77.0636) (width 0.25) (layer "B.Cu") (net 2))
 (segment (start 148.59 83.2104) (end 148.59 76.9112) (width 0.25) (layer "B.Cu") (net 2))
 (segment (start 137.668 76.9112) (end 137.668 69.9008) (width 0.25) (layer "B.Cu") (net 2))
 (segment (start 148.4376 77.0636) (end 137.8204 77.0636) (width 0.25) (layer "B.Cu") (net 2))
 (segment (start 135.128 67.216) (end 146.2908 67.216) (width 0.25) (layer "F.Cu") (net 3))
 (segment (start 146.2908 67.216) (end 146.6596 66.8472) (width 0.25) (layer "F.Cu") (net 3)))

